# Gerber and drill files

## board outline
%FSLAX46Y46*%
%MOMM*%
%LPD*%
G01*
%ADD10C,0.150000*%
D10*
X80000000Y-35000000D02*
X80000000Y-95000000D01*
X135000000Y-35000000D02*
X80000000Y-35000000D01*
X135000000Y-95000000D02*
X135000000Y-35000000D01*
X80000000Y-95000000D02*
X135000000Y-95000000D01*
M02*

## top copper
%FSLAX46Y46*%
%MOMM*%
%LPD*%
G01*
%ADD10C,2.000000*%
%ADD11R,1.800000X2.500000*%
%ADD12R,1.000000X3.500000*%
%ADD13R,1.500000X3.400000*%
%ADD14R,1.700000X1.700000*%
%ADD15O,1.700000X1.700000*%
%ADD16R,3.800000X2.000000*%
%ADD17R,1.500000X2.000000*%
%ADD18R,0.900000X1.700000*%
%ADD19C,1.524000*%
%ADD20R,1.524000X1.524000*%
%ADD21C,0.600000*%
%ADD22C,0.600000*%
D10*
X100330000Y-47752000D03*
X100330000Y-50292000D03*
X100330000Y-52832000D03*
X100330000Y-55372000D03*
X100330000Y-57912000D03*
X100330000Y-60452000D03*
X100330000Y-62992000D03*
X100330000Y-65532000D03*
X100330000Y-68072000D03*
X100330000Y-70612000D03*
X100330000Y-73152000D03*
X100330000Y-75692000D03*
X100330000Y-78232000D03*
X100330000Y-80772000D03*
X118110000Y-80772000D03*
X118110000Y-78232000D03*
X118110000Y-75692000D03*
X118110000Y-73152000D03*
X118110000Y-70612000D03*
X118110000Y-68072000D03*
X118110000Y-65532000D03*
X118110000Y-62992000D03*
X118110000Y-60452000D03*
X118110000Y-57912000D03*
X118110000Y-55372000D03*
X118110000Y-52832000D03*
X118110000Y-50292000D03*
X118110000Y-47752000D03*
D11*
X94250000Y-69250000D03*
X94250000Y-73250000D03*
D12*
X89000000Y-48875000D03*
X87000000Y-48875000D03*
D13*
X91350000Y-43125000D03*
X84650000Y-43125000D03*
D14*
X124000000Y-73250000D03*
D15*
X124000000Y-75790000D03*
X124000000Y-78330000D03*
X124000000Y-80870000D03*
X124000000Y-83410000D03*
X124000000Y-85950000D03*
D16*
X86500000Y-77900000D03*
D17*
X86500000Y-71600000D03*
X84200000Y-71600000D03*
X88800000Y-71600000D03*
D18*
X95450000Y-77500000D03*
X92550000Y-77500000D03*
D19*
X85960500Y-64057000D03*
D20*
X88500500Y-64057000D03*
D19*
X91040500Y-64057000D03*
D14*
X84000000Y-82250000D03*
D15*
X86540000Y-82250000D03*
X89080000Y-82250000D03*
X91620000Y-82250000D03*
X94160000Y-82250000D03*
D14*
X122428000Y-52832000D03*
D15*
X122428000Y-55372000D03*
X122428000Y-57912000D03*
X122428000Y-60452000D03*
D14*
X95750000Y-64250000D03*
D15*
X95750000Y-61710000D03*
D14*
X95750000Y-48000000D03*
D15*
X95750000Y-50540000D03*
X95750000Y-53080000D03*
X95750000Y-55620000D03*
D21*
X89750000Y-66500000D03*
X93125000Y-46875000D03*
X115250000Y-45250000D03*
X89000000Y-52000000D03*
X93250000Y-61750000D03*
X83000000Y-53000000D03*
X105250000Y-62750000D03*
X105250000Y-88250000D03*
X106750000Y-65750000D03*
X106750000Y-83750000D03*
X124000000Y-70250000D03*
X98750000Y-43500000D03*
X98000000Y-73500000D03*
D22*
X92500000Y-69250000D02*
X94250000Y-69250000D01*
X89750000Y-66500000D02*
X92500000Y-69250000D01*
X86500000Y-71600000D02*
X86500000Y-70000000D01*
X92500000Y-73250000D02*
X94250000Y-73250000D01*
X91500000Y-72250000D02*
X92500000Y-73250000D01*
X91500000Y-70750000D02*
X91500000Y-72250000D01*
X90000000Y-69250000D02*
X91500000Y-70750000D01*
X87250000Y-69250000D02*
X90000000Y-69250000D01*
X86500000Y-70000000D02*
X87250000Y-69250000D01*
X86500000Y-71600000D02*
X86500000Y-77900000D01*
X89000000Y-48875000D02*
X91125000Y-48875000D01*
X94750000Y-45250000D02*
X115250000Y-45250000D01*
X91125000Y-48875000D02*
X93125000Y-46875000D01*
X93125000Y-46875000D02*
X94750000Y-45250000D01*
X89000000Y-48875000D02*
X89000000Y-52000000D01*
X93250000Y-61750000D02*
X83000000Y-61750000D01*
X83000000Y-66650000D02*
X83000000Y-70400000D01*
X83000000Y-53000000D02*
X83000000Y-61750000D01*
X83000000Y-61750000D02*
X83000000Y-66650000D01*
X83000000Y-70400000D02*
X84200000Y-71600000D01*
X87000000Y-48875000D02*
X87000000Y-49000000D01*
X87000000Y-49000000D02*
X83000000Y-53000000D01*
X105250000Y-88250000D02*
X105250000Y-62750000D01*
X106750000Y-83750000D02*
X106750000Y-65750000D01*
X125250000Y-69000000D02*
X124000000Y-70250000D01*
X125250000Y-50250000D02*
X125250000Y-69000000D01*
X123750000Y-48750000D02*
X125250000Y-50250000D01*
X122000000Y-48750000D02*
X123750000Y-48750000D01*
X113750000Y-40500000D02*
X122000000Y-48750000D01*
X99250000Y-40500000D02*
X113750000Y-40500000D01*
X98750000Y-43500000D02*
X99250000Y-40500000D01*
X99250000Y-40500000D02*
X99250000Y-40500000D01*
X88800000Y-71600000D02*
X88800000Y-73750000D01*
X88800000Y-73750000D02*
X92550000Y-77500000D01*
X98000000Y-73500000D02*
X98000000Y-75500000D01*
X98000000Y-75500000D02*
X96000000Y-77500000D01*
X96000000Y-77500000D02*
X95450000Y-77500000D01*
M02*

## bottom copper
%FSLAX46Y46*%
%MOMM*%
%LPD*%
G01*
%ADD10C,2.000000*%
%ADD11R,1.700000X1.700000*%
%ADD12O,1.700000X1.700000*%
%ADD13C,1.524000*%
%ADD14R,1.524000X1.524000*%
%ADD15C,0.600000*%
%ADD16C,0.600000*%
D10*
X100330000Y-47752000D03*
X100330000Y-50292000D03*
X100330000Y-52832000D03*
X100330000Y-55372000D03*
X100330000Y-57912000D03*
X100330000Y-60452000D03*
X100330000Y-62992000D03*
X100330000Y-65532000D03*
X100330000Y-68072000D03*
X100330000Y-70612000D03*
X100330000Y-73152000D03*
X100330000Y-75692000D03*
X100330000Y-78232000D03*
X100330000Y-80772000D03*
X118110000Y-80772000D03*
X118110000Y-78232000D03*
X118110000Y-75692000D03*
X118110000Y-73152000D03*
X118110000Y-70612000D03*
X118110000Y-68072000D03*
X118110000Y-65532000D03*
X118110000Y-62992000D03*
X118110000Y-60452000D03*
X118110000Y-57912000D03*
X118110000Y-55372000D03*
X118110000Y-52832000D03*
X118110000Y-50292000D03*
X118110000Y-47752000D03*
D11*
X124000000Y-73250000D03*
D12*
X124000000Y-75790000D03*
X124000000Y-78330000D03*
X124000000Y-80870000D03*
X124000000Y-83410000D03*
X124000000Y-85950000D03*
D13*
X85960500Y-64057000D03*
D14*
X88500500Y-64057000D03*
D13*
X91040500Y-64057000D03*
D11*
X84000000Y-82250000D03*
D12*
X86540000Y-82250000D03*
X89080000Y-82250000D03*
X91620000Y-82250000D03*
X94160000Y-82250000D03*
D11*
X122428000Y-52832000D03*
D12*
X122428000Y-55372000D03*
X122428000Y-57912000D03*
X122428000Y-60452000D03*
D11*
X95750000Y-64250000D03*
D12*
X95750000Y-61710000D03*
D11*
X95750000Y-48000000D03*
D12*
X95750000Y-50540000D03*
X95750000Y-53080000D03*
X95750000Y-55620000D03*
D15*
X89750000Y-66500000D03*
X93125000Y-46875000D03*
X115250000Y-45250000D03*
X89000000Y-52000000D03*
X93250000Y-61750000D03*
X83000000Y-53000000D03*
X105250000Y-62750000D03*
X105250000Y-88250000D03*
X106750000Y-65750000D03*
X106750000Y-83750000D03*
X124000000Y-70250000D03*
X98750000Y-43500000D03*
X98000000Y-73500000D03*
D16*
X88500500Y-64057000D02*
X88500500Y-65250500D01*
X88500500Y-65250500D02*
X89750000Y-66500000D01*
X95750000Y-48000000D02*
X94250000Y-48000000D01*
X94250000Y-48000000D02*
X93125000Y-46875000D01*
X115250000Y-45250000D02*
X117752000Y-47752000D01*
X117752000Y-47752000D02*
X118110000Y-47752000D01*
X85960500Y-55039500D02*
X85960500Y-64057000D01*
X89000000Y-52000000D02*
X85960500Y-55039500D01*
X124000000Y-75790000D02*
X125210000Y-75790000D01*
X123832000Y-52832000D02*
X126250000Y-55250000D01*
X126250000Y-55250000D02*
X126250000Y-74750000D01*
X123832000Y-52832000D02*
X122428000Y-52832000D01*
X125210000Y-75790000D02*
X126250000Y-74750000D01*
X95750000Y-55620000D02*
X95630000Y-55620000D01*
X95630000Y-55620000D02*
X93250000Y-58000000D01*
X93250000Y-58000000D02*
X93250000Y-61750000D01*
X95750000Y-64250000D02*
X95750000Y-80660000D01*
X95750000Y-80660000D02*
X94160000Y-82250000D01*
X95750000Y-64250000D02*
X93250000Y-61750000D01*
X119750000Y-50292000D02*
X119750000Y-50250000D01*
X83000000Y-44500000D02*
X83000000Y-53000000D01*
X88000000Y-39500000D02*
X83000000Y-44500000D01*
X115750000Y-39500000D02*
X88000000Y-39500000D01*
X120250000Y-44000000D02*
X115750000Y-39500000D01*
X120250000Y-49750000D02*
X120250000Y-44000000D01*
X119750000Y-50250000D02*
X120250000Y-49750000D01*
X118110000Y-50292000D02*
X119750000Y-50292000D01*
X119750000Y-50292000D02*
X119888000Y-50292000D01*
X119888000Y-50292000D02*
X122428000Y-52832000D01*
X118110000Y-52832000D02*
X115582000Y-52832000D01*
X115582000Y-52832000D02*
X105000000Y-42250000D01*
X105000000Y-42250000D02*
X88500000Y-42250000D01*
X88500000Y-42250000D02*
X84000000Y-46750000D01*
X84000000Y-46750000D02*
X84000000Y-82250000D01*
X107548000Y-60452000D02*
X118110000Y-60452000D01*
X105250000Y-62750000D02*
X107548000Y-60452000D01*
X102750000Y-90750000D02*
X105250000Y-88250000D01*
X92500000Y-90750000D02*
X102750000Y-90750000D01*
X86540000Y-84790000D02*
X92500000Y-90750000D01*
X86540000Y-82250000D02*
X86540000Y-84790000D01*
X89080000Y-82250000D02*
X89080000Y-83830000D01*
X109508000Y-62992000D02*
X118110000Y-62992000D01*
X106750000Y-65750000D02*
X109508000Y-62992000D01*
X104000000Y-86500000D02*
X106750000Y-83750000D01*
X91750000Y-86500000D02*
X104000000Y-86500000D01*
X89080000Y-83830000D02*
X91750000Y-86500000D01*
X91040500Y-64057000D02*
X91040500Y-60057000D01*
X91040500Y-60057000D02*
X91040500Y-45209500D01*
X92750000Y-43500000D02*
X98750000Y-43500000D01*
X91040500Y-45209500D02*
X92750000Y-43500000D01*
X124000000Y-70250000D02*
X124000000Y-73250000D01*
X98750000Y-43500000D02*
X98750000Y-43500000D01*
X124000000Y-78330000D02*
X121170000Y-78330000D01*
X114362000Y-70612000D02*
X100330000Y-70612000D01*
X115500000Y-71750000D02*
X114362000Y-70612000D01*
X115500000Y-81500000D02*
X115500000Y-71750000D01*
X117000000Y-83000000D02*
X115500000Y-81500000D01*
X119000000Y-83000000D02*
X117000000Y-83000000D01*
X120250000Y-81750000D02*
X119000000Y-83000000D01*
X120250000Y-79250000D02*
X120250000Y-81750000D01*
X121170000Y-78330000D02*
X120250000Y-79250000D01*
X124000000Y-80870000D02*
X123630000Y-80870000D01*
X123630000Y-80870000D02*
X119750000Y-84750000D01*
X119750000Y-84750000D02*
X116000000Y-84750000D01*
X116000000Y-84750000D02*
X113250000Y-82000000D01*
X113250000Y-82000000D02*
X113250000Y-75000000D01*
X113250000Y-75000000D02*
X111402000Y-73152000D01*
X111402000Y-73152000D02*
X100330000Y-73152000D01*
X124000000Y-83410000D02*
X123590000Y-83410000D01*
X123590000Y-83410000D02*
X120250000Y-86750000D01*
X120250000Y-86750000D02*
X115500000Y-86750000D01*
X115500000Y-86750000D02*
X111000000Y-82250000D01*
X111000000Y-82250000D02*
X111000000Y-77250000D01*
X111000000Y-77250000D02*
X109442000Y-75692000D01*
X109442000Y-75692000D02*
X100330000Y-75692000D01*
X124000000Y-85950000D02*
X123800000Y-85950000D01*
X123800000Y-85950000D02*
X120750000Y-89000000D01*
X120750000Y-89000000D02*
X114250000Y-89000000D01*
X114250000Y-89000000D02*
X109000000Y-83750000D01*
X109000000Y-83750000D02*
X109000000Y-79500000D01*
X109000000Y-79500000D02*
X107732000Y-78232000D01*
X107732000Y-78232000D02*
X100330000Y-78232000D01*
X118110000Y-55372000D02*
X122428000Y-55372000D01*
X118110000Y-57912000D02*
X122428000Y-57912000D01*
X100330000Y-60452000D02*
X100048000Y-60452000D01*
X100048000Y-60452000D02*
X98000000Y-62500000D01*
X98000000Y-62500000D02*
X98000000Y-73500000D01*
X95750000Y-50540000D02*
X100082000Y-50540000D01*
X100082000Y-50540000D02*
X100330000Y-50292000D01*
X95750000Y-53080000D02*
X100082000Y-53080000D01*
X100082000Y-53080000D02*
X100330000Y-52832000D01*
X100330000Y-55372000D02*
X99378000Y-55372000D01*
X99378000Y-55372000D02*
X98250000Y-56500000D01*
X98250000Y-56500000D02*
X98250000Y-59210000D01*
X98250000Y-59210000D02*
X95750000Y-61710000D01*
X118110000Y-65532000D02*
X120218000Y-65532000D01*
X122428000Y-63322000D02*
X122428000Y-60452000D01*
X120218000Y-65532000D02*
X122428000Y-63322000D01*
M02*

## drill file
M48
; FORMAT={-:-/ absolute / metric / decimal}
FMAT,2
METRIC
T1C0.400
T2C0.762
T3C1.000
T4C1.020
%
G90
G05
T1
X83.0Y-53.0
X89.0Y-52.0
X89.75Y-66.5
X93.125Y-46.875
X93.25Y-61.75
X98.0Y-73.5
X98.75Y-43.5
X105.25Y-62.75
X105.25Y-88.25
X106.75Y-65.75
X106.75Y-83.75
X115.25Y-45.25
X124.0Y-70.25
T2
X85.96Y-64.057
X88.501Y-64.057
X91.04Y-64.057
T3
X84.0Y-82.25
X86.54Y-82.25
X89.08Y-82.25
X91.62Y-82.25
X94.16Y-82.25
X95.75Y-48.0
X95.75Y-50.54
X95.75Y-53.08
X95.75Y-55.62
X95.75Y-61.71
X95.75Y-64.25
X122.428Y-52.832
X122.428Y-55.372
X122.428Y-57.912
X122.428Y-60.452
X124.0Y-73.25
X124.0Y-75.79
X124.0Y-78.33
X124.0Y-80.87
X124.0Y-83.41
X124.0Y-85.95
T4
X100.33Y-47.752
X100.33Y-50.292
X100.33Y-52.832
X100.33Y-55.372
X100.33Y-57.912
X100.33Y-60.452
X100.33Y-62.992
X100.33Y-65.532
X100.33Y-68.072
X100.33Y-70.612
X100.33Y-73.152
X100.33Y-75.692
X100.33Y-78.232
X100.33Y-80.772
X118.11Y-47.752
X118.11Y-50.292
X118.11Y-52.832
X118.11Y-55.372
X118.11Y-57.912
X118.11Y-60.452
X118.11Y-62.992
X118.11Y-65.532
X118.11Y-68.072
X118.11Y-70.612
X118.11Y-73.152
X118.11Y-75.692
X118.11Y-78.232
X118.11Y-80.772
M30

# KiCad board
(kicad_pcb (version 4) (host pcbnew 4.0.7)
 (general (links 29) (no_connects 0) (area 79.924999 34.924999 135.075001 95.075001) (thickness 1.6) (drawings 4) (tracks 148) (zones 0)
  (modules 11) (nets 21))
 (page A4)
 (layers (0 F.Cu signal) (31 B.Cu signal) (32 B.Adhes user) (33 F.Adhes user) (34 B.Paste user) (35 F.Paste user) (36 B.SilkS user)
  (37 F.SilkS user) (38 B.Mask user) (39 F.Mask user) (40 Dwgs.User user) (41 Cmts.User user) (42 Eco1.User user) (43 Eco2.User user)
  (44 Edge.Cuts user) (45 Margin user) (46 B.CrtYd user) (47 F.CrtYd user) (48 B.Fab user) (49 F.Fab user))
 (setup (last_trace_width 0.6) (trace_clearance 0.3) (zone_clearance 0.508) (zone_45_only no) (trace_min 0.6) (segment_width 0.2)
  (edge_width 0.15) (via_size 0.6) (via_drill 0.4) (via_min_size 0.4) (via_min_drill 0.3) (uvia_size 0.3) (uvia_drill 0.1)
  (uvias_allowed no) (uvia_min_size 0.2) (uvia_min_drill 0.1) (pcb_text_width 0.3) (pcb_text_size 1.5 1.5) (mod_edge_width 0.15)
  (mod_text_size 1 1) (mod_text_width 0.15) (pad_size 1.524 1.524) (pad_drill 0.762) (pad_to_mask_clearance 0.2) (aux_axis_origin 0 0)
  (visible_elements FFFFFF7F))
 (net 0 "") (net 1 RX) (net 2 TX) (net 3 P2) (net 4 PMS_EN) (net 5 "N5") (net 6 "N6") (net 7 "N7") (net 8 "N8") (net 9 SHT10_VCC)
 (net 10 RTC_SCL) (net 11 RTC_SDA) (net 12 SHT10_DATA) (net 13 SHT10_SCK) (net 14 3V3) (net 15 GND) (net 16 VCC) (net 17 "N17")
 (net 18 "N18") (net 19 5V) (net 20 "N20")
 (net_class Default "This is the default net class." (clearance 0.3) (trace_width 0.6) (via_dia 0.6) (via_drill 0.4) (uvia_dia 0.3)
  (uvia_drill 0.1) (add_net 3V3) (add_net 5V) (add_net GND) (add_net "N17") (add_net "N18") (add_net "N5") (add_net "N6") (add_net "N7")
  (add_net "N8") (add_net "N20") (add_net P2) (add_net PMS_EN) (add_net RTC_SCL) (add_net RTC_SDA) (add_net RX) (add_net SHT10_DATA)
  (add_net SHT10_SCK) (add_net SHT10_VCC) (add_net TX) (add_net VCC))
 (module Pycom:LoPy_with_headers (layer F.Cu) (at 100.33 47.752 270)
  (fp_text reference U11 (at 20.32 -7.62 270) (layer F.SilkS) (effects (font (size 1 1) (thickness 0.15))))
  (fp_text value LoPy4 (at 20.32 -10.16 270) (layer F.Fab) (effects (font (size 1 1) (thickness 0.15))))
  (pad 1 thru_hole circle (at 0 0 270) (size 2 2) (drill 1.02) (layers *.Cu *.Mask))
  (pad 2 thru_hole circle (at 2.54 0 270) (size 2 2) (drill 1.02) (layers *.Cu *.Mask) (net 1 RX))
  (pad 3 thru_hole circle (at 5.08 0 270) (size 2 2) (drill 1.02) (layers *.Cu *.Mask) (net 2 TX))
  (pad 4 thru_hole circle (at 7.62 0 270) (size 2 2) (drill 1.02) (layers *.Cu *.Mask) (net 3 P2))
  (pad 5 thru_hole circle (at 10.16 0 270) (size 2 2) (drill 1.02) (layers *.Cu *.Mask))
  (pad 6 thru_hole circle (at 12.7 0 270) (size 2 2) (drill 1.02) (layers *.Cu *.Mask) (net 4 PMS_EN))
  (pad 7 thru_hole circle (at 15.24 0 270) (size 2 2) (drill 1.02) (layers *.Cu *.Mask))
  (pad 8 thru_hole circle (at 17.78 0 270) (size 2 2) (drill 1.02) (layers *.Cu *.Mask))
  (pad 9 thru_hole circle (at 20.32 0 270) (size 2 2) (drill 1.02) (layers *.Cu *.Mask))
  (pad 10 thru_hole circle (at 22.86 0 270) (size 2 2) (drill 1.02) (layers *.Cu *.Mask) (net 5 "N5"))
  (pad 11 thru_hole circle (at 25.4 0 270) (size 2 2) (drill 1.02) (layers *.Cu *.Mask) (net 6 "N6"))
  (pad 12 thru_hole circle (at 27.94 0 270) (size 2 2) (drill 1.02) (layers *.Cu *.Mask) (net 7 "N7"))
  (pad 13 thru_hole circle (at 30.48 0 270) (size 2 2) (drill 1.02) (layers *.Cu *.Mask) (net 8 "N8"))
  (pad 14 thru_hole circle (at 33.02 0 270) (size 2 2) (drill 1.02) (layers *.Cu *.Mask))
  (pad 15 thru_hole circle (at 33.02 -17.78 270) (size 2 2) (drill 1.02) (layers *.Cu *.Mask))
  (pad 16 thru_hole circle (at 30.48 -17.78 270) (size 2 2) (drill 1.02) (layers *.Cu *.Mask))
  (pad 17 thru_hole circle (at 27.94 -17.78 270) (size 2 2) (drill 1.02) (layers *.Cu *.Mask))
  (pad 18 thru_hole circle (at 25.4 -17.78 270) (size 2 2) (drill 1.02) (layers *.Cu *.Mask))
  (pad 19 thru_hole circle (at 22.86 -17.78 270) (size 2 2) (drill 1.02) (layers *.Cu *.Mask))
  (pad 20 thru_hole circle (at 20.32 -17.78 270) (size 2 2) (drill 1.02) (layers *.Cu *.Mask))
  (pad 21 thru_hole circle (at 17.78 -17.78 270) (size 2 2) (drill 1.02) (layers *.Cu *.Mask) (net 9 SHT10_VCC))
  (pad 22 thru_hole circle (at 15.24 -17.78 270) (size 2 2) (drill 1.02) (layers *.Cu *.Mask) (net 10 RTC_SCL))
  (pad 23 thru_hole circle (at 12.7 -17.78 270) (size 2 2) (drill 1.02) (layers *.Cu *.Mask) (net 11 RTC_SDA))
  (pad 24 thru_hole circle (at 10.16 -17.78 270) (size 2 2) (drill 1.02) (layers *.Cu *.Mask) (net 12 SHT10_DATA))
  (pad 25 thru_hole circle (at 7.62 -17.78 270) (size 2 2) (drill 1.02) (layers *.Cu *.Mask) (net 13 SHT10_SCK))
  (pad 26 thru_hole circle (at 5.08 -17.78 270) (size 2 2) (drill 1.02) (layers *.Cu *.Mask) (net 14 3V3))
  (pad 27 thru_hole circle (at 2.54 -17.78 270) (size 2 2) (drill 1.02) (layers *.Cu *.Mask) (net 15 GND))
  (pad 28 thru_hole circle (at 0 -17.78 270) (size 2 2) (drill 1.02) (layers *.Cu *.Mask) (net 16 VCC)))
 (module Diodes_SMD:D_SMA (layer F.Cu) (at 94.25 71.25 270)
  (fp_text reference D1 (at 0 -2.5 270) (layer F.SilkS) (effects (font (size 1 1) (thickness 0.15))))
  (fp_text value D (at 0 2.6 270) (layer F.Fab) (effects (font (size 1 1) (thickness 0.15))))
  (pad 1 smd rect (at -2 0 270) (size 2.5 1.8) (layers F.Cu F.Paste F.Mask) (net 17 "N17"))
  (pad 2 smd rect (at 2 0 270) (size 2.5 1.8) (layers F.Cu F.Paste F.Mask) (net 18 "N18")))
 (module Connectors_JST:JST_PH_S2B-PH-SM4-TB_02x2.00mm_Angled (layer F.Cu) (at 88 46 180)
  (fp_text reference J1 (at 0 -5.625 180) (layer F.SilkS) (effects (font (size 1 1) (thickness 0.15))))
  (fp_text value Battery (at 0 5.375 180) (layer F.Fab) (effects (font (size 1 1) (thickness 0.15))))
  (pad 1 smd rect (at -1 -2.875 180) (size 1 3.5) (layers F.Cu F.Paste F.Mask) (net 16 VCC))
  (pad 2 smd rect (at 1 -2.875 180) (size 1 3.5) (layers F.Cu F.Paste F.Mask) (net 15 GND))
  (pad "" smd rect (at -3.35 2.875 180) (size 1.5 3.4) (layers F.Cu F.Paste F.Mask))
  (pad "" smd rect (at 3.35 2.875 180) (size 1.5 3.4) (layers F.Cu F.Paste F.Mask)))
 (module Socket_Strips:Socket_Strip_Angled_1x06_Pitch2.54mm (layer B.Cu) (at 124 73.25 180)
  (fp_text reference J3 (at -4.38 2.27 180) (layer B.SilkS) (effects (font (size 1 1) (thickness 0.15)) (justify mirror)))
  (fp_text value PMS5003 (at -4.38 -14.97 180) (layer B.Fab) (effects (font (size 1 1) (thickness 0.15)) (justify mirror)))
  (pad 1 thru_hole rect (at 0 0 180) (size 1.7 1.7) (drill 1) (layers *.Cu *.Mask) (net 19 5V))
  (pad 2 thru_hole oval (at 0 -2.54 180) (size 1.7 1.7) (drill 1) (layers *.Cu *.Mask) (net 15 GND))
  (pad 3 thru_hole oval (at 0 -5.08 180) (size 1.7 1.7) (drill 1) (layers *.Cu *.Mask) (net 5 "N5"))
  (pad 4 thru_hole oval (at 0 -7.62 180) (size 1.7 1.7) (drill 1) (layers *.Cu *.Mask) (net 6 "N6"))
  (pad 5 thru_hole oval (at 0 -10.16 180) (size 1.7 1.7) (drill 1) (layers *.Cu *.Mask) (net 7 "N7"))
  (pad 6 thru_hole oval (at 0 -12.7 180) (size 1.7 1.7) (drill 1) (layers *.Cu *.Mask) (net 8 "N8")))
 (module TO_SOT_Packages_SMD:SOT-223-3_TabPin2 (layer F.Cu) (at 86.5 74.75 270)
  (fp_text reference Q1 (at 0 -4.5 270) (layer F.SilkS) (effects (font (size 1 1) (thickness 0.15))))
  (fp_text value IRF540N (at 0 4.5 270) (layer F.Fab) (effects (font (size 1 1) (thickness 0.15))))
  (pad 2 smd rect (at 3.15 0 270) (size 2 3.8) (layers F.Cu F.Paste F.Mask) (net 18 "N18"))
  (pad 2 smd rect (at -3.15 0 270) (size 2 1.5) (layers F.Cu F.Paste F.Mask) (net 18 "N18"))
  (pad 3 smd rect (at -3.15 2.3 270) (size 2 1.5) (layers F.Cu F.Paste F.Mask) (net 15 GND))
  (pad 1 smd rect (at -3.15 -2.3 270) (size 2 1.5) (layers F.Cu F.Paste F.Mask) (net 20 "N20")))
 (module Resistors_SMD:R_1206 (layer F.Cu) (at 94 77.5 180)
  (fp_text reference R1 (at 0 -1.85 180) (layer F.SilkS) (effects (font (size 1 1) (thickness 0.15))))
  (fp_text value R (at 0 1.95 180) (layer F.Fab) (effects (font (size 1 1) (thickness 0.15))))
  (pad 1 smd rect (at -1.45 0 180) (size 0.9 1.7) (layers F.Cu F.Paste F.Mask) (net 4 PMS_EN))
  (pad 2 smd rect (at 1.45 0 180) (size 0.9 1.7) (layers F.Cu F.Paste F.Mask) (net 20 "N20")))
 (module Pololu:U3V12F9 (layer F.Cu) (at 84.5 52.5 270)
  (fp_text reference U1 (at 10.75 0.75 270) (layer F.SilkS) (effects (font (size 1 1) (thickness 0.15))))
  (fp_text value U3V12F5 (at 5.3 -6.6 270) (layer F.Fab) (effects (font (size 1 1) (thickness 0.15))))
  (pad 1 thru_hole circle (at 11.557 -1.4605 270) (size 1.524 1.524) (drill 0.762) (layers *.Cu *.Mask) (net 16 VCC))
  (pad 2 thru_hole rect (at 11.557 -4.0005 270) (size 1.524 1.524) (drill 0.762) (layers *.Cu *.Mask) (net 17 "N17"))
  (pad 3 thru_hole circle (at 11.557 -6.5405 270) (size 1.524 1.524) (drill 0.762) (layers *.Cu *.Mask) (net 19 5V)))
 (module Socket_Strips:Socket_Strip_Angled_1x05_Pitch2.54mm (layer F.Cu) (at 84 82.25 90)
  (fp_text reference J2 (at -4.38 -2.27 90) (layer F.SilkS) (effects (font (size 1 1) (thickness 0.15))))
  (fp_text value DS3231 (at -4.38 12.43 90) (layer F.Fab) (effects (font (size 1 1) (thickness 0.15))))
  (pad 1 thru_hole rect (at 0 0 90) (size 1.7 1.7) (drill 1) (layers *.Cu *.Mask) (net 14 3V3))
  (pad 2 thru_hole oval (at 0 2.54 90) (size 1.7 1.7) (drill 1) (layers *.Cu *.Mask) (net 11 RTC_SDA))
  (pad 3 thru_hole oval (at 0 5.08 90) (size 1.7 1.7) (drill 1) (layers *.Cu *.Mask) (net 10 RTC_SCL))
  (pad 4 thru_hole oval (at 0 7.62 90) (size 1.7 1.7) (drill 1) (layers *.Cu *.Mask))
  (pad 5 thru_hole oval (at 0 10.16 90) (size 1.7 1.7) (drill 1) (layers *.Cu *.Mask) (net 15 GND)))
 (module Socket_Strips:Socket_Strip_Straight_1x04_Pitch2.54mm (layer F.Cu) (at 122.428 52.832)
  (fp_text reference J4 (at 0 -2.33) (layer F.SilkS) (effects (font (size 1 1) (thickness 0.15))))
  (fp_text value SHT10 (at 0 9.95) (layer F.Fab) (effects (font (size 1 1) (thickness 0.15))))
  (pad 1 thru_hole rect (at 0 0) (size 1.7 1.7) (drill 1) (layers *.Cu *.Mask) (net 15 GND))
  (pad 2 thru_hole oval (at 0 2.54) (size 1.7 1.7) (drill 1) (layers *.Cu *.Mask) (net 13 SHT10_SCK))
  (pad 3 thru_hole oval (at 0 5.08) (size 1.7 1.7) (drill 1) (layers *.Cu *.Mask) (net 12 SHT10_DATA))
  (pad 4 thru_hole oval (at 0 7.62) (size 1.7 1.7) (drill 1) (layers *.Cu *.Mask) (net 9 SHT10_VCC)))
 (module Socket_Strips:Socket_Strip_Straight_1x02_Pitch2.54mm (layer F.Cu) (at 95.75 64.25 180)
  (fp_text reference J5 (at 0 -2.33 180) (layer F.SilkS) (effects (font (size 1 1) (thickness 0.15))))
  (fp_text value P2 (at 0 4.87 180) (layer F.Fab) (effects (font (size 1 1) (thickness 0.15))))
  (pad 1 thru_hole rect (at 0 0 180) (size 1.7 1.7) (drill 1) (layers *.Cu *.Mask) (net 15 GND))
  (pad 2 thru_hole oval (at 0 2.54 180) (size 1.7 1.7) (drill 1) (layers *.Cu *.Mask) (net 3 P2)))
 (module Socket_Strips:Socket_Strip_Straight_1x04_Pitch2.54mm (layer F.Cu) (at 95.75 48)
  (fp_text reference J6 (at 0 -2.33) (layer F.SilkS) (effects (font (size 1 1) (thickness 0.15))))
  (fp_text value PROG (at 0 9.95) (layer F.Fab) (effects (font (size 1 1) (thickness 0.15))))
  (pad 1 thru_hole rect (at 0 0) (size 1.7 1.7) (drill 1) (layers *.Cu *.Mask) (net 16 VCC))
  (pad 2 thru_hole oval (at 0 2.54) (size 1.7 1.7) (drill 1) (layers *.Cu *.Mask) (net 1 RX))
  (pad 3 thru_hole oval (at 0 5.08) (size 1.7 1.7) (drill 1) (layers *.Cu *.Mask) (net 2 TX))
  (pad 4 thru_hole oval (at 0 7.62) (size 1.7 1.7) (drill 1) (layers *.Cu *.Mask) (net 15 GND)))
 (gr_line (start 80 35) (end 80 95) (angle 90) (layer Edge.Cuts) (width 0.15))
 (gr_line (start 135 35) (end 80 35) (angle 90) (layer Edge.Cuts) (width 0.15))
 (gr_line (start 135 95) (end 135 35) (angle 90) (layer Edge.Cuts) (width 0.15))
 (gr_line (start 80 95) (end 135 95) (angle 90) (layer Edge.Cuts) (width 0.15))
 (segment (start 88.5005 64.057) (end 88.5005 65.2505) (width 0.6) (layer B.Cu) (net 17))
 (segment (start 92.5 69.25) (end 94.25 69.25) (width 0.6) (layer F.Cu) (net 17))
 (segment (start 89.75 66.5) (end 92.5 69.25) (width 0.6) (layer F.Cu) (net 17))
 (via (at 89.75 66.5) (size 0.6) (drill 0.4) (layers F.Cu B.Cu) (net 17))
 (segment (start 88.5005 65.2505) (end 89.75 66.5) (width 0.6) (layer B.Cu) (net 17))
 (segment (start 86.5 71.6) (end 86.5 70) (width 0.6) (layer F.Cu) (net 18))
 (segment (start 92.5 73.25) (end 94.25 73.25) (width 0.6) (layer F.Cu) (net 18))
 (segment (start 91.5 72.25) (end 92.5 73.25) (width 0.6) (layer F.Cu) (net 18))
 (segment (start 91.5 70.75) (end 91.5 72.25) (width 0.6) (layer F.Cu) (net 18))
 (segment (start 90 69.25) (end 91.5 70.75) (width 0.6) (layer F.Cu) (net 18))
 (segment (start 87.25 69.25) (end 90 69.25) (width 0.6) (layer F.Cu) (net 18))
 (segment (start 86.5 70) (end 87.25 69.25) (width 0.6) (layer F.Cu) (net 18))
 (segment (start 86.5 71.6) (end 86.5 77.9) (width 0.6) (layer F.Cu) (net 18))
 (via (at 93.125 46.875) (size 0.6) (drill 0.4) (layers F.Cu B.Cu) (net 16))
 (segment (start 95.75 48) (end 94.25 48) (width 0.6) (layer B.Cu) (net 16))
 (segment (start 94.25 48) (end 93.125 46.875) (width 0.6) (layer B.Cu) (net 16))
 (segment (start 89 48.875) (end 91.125 48.875) (width 0.6) (layer F.Cu) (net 16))
 (segment (start 115.25 45.25) (end 117.752 47.752) (width 0.6) (layer B.Cu) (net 16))
 (via (at 115.25 45.25) (size 0.6) (drill 0.4) (layers F.Cu B.Cu) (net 16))
 (segment (start 94.75 45.25) (end 115.25 45.25) (width 0.6) (layer F.Cu) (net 16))
 (segment (start 91.125 48.875) (end 93.125 46.875) (width 0.6) (layer F.Cu) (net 16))
 (segment (start 93.125 46.875) (end 94.75 45.25) (width 0.6) (layer F.Cu) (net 16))
 (segment (start 117.752 47.752) (end 118.11 47.752) (width 0.6) (layer B.Cu) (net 16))
 (segment (start 89 48.875) (end 89 52) (width 0.6) (layer F.Cu) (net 16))
 (segment (start 85.9605 55.0395) (end 85.9605 64.057) (width 0.6) (layer B.Cu) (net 16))
 (segment (start 89 52) (end 85.9605 55.0395) (width 0.6) (layer B.Cu) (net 16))
 (via (at 89 52) (size 0.6) (drill 0.4) (layers F.Cu B.Cu) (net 16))
 (segment (start 124 75.79) (end 125.21 75.79) (width 0.6) (layer B.Cu) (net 15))
 (segment (start 123.832 52.832) (end 126.25 55.25) (width 0.6) (layer B.Cu) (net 15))
 (segment (start 126.25 55.25) (end 126.25 74.75) (width 0.6) (layer B.Cu) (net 15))
 (segment (start 123.832 52.832) (end 122.428 52.832) (width 0.6) (layer B.Cu) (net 15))
 (segment (start 125.21 75.79) (end 126.25 74.75) (width 0.6) (layer B.Cu) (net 15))
 (segment (start 95.75 55.62) (end 95.63 55.62) (width 0.6) (layer B.Cu) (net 15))
 (segment (start 95.63 55.62) (end 93.25 58) (width 0.6) (layer B.Cu) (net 15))
 (segment (start 93.25 58) (end 93.25 61.75) (width 0.6) (layer B.Cu) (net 15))
 (segment (start 95.75 64.25) (end 95.75 80.66) (width 0.6) (layer B.Cu) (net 15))
 (segment (start 95.75 80.66) (end 94.16 82.25) (width 0.6) (layer B.Cu) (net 15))
 (segment (start 95.75 64.25) (end 93.25 61.75) (width 0.6) (layer B.Cu) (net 15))
 (segment (start 93.25 61.75) (end 83 61.75) (width 0.6) (layer F.Cu) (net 15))
 (via (at 93.25 61.75) (size 0.6) (drill 0.4) (layers F.Cu B.Cu) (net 15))
 (segment (start 83 66.65) (end 83 70.4) (width 0.6) (layer F.Cu) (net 15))
 (segment (start 83 53) (end 83 61.75) (width 0.6) (layer F.Cu) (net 15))
 (segment (start 83 61.75) (end 83 66.65) (width 0.6) (layer F.Cu) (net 15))
 (segment (start 83 70.4) (end 84.2 71.6) (width 0.6) (layer F.Cu) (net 15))
 (segment (start 119.75 50.292) (end 119.75 50.25) (width 0.6) (layer B.Cu) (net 15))
 (via (at 83 53) (size 0.6) (drill 0.4) (layers F.Cu B.Cu) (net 15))
 (segment (start 83 44.5) (end 83 53) (width 0.6) (layer B.Cu) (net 15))
 (segment (start 88 39.5) (end 83 44.5) (width 0.6) (layer B.Cu) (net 15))
 (segment (start 115.75 39.5) (end 88 39.5) (width 0.6) (layer B.Cu) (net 15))
 (segment (start 120.25 44) (end 115.75 39.5) (width 0.6) (layer B.Cu) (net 15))
 (segment (start 120.25 49.75) (end 120.25 44) (width 0.6) (layer B.Cu) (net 15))
 (segment (start 119.75 50.25) (end 120.25 49.75) (width 0.6) (layer B.Cu) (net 15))
 (segment (start 118.11 50.292) (end 119.75 50.292) (width 0.6) (layer B.Cu) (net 15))
 (segment (start 119.75 50.292) (end 119.888 50.292) (width 0.6) (layer B.Cu) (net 15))
 (segment (start 119.888 50.292) (end 122.428 52.832) (width 0.6) (layer B.Cu) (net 15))
 (segment (start 87 48.875) (end 87 49) (width 0.6) (layer F.Cu) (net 15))
 (segment (start 87 49) (end 83 53) (width 0.6) (layer F.Cu) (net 15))
 (segment (start 118.11 52.832) (end 115.582 52.832) (width 0.6) (layer B.Cu) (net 14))
 (segment (start 115.582 52.832) (end 105 42.25) (width 0.6) (layer B.Cu) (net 14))
 (segment (start 105 42.25) (end 88.5 42.25) (width 0.6) (layer B.Cu) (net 14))
 (segment (start 88.5 42.25) (end 84 46.75) (width 0.6) (layer B.Cu) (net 14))
 (segment (start 84 46.75) (end 84 82.25) (width 0.6) (layer B.Cu) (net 14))
 (segment (start 107.548 60.452) (end 118.11 60.452) (width 0.6) (layer B.Cu) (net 11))
 (segment (start 105.25 62.75) (end 107.548 60.452) (width 0.6) (layer B.Cu) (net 11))
 (via (at 105.25 62.75) (size 0.6) (drill 0.4) (layers F.Cu B.Cu) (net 11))
 (segment (start 105.25 88.25) (end 105.25 62.75) (width 0.6) (layer F.Cu) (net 11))
 (via (at 105.25 88.25) (size 0.6) (drill 0.4) (layers F.Cu B.Cu) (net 11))
 (segment (start 102.75 90.75) (end 105.25 88.25) (width 0.6) (layer B.Cu) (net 11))
 (segment (start 92.5 90.75) (end 102.75 90.75) (width 0.6) (layer B.Cu) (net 11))
 (segment (start 86.54 84.79) (end 92.5 90.75) (width 0.6) (layer B.Cu) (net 11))
 (segment (start 86.54 82.25) (end 86.54 84.79) (width 0.6) (layer B.Cu) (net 11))
 (segment (start 89.08 82.25) (end 89.08 83.83) (width 0.6) (layer B.Cu) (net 10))
 (segment (start 109.508 62.992) (end 118.11 62.992) (width 0.6) (layer B.Cu) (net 10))
 (segment (start 106.75 65.75) (end 109.508 62.992) (width 0.6) (layer B.Cu) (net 10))
 (via (at 106.75 65.75) (size 0.6) (drill 0.4) (layers F.Cu B.Cu) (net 10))
 (segment (start 106.75 83.75) (end 106.75 65.75) (width 0.6) (layer F.Cu) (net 10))
 (via (at 106.75 83.75) (size 0.6) (drill 0.4) (layers F.Cu B.Cu) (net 10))
 (segment (start 104 86.5) (end 106.75 83.75) (width 0.6) (layer B.Cu) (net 10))
 (segment (start 91.75 86.5) (end 104 86.5) (width 0.6) (layer B.Cu) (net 10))
 (segment (start 89.08 83.83) (end 91.75 86.5) (width 0.6) (layer B.Cu) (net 10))
 (segment (start 91.0405 64.057) (end 91.0405 60.057) (width 0.6) (layer B.Cu) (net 19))
 (segment (start 91.0405 60.057) (end 91.0405 45.2095) (width 0.6) (layer B.Cu) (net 19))
 (segment (start 92.75 43.5) (end 98.75 43.5) (width 0.6) (layer B.Cu) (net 19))
 (segment (start 91.0405 45.2095) (end 92.75 43.5) (width 0.6) (layer B.Cu) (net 19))
 (segment (start 124 70.25) (end 124 73.25) (width 0.6) (layer B.Cu) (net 19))
 (via (at 124 70.25) (size 0.6) (drill 0.4) (layers F.Cu B.Cu) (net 19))
 (segment (start 125.25 69) (end 124 70.25) (width 0.6) (layer F.Cu) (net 19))
 (segment (start 125.25 50.25) (end 125.25 69) (width 0.6) (layer F.Cu) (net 19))
 (segment (start 123.75 48.75) (end 125.25 50.25) (width 0.6) (layer F.Cu) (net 19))
 (segment (start 122 48.75) (end 123.75 48.75) (width 0.6) (layer F.Cu) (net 19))
 (segment (start 113.75 40.5) (end 122 48.75) (width 0.6) (layer F.Cu) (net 19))
 (segment (start 99.25 40.5) (end 113.75 40.5) (width 0.6) (layer F.Cu) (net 19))
 (segment (start 98.75 43.5) (end 98.75 43.5) (width 0.6) (layer B.Cu) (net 19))
 (via (at 98.75 43.5) (size 0.6) (drill 0.4) (layers F.Cu B.Cu) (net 19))
 (segment (start 98.75 43.5) (end 99.25 40.5) (width 0.6) (layer F.Cu) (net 19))
 (segment (start 99.25 40.5) (end 99.25 40.5) (width 0.6) (layer F.Cu) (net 19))
 (segment (start 124 78.33) (end 121.17 78.33) (width 0.6) (layer B.Cu) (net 5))
 (segment (start 114.362 70.612) (end 100.33 70.612) (width 0.6) (layer B.Cu) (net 5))
 (segment (start 115.5 71.75) (end 114.362 70.612) (width 0.6) (layer B.Cu) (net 5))
 (segment (start 115.5 81.5) (end 115.5 71.75) (width 0.6) (layer B.Cu) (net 5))
 (segment (start 117 83) (end 115.5 81.5) (width 0.6) (layer B.Cu) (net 5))
 (segment (start 119 83) (end 117 83) (width 0.6) (layer B.Cu) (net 5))
 (segment (start 120.25 81.75) (end 119 83) (width 0.6) (layer B.Cu) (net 5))
 (segment (start 120.25 79.25) (end 120.25 81.75) (width 0.6) (layer B.Cu) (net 5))
 (segment (start 121.17 78.33) (end 120.25 79.25) (width 0.6) (layer B.Cu) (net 5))
 (segment (start 124 80.87) (end 123.63 80.87) (width 0.6) (layer B.Cu) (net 6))
 (segment (start 123.63 80.87) (end 119.75 84.75) (width 0.6) (layer B.Cu) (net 6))
 (segment (start 119.75 84.75) (end 116 84.75) (width 0.6) (layer B.Cu) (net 6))
 (segment (start 116 84.75) (end 113.25 82) (width 0.6) (layer B.Cu) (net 6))
 (segment (start 113.25 82) (end 113.25 75) (width 0.6) (layer B.Cu) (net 6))
 (segment (start 113.25 75) (end 111.402 73.152) (width 0.6) (layer B.Cu) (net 6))
 (segment (start 111.402 73.152) (end 100.33 73.152) (width 0.6) (layer B.Cu) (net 6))
 (segment (start 124 83.41) (end 123.59 83.41) (width 0.6) (layer B.Cu) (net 7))
 (segment (start 123.59 83.41) (end 120.25 86.75) (width 0.6) (layer B.Cu) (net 7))
 (segment (start 120.25 86.75) (end 115.5 86.75) (width 0.6) (layer B.Cu) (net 7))
 (segment (start 115.5 86.75) (end 111 82.25) (width 0.6) (layer B.Cu) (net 7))
 (segment (start 111 82.25) (end 111 77.25) (width 0.6) (layer B.Cu) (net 7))
 (segment (start 111 77.25) (end 109.442 75.692) (width 0.6) (layer B.Cu) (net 7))
 (segment (start 109.442 75.692) (end 100.33 75.692) (width 0.6) (layer B.Cu) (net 7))
 (segment (start 124 85.95) (end 123.8 85.95) (width 0.6) (layer B.Cu) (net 8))
 (segment (start 123.8 85.95) (end 120.75 89) (width 0.6) (layer B.Cu) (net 8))
 (segment (start 120.75 89) (end 114.25 89) (width 0.6) (layer B.Cu) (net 8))
 (segment (start 114.25 89) (end 109 83.75) (width 0.6) (layer B.Cu) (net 8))
 (segment (start 109 83.75) (end 109 79.5) (width 0.6) (layer B.Cu) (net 8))
 (segment (start 109 79.5) (end 107.732 78.232) (width 0.6) (layer B.Cu) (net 8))
 (segment (start 107.732 78.232) (end 100.33 78.232) (width 0.6) (layer B.Cu) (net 8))
 (segment (start 118.11 55.372) (end 122.428 55.372) (width 0.6) (layer B.Cu) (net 13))
 (segment (start 118.11 57.912) (end 122.428 57.912) (width 0.6) (layer B.Cu) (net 12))
 (segment (start 88.8 71.6) (end 88.8 73.75) (width 0.6) (layer F.Cu) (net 20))
 (segment (start 88.8 73.75) (end 92.55 77.5) (width 0.6) (layer F.Cu) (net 20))
 (segment (start 100.33 60.452) (end 100.048 60.452) (width 0.6) (layer B.Cu) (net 4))
 (segment (start 100.048 60.452) (end 98 62.5) (width 0.6) (layer B.Cu) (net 4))
 (segment (start 98 62.5) (end 98 73.5) (width 0.6) (layer B.Cu) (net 4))
 (via (at 98 73.5) (size 0.6) (drill 0.4) (layers F.Cu B.Cu) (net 4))
 (segment (start 98 73.5) (end 98 75.5) (width 0.6) (layer F.Cu) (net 4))
 (segment (start 98 75.5) (end 96 77.5) (width 0.6) (layer F.Cu) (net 4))
 (segment (start 96 77.5) (end 95.45 77.5) (width 0.6) (layer F.Cu) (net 4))
 (segment (start 95.75 50.54) (end 100.082 50.54) (width 0.6) (layer B.Cu) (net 1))
 (segment (start 100.082 50.54) (end 100.33 50.292) (width 0.6) (layer B.Cu) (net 1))
 (segment (start 95.75 53.08) (end 100.082 53.08) (width 0.6) (layer B.Cu) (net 2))
 (segment (start 100.082 53.08) (end 100.33 52.832) (width 0.6) (layer B.Cu) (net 2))
 (segment (start 100.33 55.372) (end 99.378 55.372) (width 0.6) (layer B.Cu) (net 3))
 (segment (start 99.378 55.372) (end 98.25 56.5) (width 0.6) (layer B.Cu) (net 3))
 (segment (start 98.25 56.5) (end 98.25 59.21) (width 0.6) (layer B.Cu) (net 3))
 (segment (start 98.25 59.21) (end 95.75 61.71) (width 0.6) (layer B.Cu) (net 3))
 (segment (start 118.11 65.532) (end 120.218 65.532) (width 0.6) (layer B.Cu) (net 9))
 (segment (start 122.428 63.322) (end 122.428 60.452) (width 0.6) (layer B.Cu) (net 9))
 (segment (start 120.218 65.532) (end 122.428 63.322) (width 0.6) (layer B.Cu) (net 9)))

